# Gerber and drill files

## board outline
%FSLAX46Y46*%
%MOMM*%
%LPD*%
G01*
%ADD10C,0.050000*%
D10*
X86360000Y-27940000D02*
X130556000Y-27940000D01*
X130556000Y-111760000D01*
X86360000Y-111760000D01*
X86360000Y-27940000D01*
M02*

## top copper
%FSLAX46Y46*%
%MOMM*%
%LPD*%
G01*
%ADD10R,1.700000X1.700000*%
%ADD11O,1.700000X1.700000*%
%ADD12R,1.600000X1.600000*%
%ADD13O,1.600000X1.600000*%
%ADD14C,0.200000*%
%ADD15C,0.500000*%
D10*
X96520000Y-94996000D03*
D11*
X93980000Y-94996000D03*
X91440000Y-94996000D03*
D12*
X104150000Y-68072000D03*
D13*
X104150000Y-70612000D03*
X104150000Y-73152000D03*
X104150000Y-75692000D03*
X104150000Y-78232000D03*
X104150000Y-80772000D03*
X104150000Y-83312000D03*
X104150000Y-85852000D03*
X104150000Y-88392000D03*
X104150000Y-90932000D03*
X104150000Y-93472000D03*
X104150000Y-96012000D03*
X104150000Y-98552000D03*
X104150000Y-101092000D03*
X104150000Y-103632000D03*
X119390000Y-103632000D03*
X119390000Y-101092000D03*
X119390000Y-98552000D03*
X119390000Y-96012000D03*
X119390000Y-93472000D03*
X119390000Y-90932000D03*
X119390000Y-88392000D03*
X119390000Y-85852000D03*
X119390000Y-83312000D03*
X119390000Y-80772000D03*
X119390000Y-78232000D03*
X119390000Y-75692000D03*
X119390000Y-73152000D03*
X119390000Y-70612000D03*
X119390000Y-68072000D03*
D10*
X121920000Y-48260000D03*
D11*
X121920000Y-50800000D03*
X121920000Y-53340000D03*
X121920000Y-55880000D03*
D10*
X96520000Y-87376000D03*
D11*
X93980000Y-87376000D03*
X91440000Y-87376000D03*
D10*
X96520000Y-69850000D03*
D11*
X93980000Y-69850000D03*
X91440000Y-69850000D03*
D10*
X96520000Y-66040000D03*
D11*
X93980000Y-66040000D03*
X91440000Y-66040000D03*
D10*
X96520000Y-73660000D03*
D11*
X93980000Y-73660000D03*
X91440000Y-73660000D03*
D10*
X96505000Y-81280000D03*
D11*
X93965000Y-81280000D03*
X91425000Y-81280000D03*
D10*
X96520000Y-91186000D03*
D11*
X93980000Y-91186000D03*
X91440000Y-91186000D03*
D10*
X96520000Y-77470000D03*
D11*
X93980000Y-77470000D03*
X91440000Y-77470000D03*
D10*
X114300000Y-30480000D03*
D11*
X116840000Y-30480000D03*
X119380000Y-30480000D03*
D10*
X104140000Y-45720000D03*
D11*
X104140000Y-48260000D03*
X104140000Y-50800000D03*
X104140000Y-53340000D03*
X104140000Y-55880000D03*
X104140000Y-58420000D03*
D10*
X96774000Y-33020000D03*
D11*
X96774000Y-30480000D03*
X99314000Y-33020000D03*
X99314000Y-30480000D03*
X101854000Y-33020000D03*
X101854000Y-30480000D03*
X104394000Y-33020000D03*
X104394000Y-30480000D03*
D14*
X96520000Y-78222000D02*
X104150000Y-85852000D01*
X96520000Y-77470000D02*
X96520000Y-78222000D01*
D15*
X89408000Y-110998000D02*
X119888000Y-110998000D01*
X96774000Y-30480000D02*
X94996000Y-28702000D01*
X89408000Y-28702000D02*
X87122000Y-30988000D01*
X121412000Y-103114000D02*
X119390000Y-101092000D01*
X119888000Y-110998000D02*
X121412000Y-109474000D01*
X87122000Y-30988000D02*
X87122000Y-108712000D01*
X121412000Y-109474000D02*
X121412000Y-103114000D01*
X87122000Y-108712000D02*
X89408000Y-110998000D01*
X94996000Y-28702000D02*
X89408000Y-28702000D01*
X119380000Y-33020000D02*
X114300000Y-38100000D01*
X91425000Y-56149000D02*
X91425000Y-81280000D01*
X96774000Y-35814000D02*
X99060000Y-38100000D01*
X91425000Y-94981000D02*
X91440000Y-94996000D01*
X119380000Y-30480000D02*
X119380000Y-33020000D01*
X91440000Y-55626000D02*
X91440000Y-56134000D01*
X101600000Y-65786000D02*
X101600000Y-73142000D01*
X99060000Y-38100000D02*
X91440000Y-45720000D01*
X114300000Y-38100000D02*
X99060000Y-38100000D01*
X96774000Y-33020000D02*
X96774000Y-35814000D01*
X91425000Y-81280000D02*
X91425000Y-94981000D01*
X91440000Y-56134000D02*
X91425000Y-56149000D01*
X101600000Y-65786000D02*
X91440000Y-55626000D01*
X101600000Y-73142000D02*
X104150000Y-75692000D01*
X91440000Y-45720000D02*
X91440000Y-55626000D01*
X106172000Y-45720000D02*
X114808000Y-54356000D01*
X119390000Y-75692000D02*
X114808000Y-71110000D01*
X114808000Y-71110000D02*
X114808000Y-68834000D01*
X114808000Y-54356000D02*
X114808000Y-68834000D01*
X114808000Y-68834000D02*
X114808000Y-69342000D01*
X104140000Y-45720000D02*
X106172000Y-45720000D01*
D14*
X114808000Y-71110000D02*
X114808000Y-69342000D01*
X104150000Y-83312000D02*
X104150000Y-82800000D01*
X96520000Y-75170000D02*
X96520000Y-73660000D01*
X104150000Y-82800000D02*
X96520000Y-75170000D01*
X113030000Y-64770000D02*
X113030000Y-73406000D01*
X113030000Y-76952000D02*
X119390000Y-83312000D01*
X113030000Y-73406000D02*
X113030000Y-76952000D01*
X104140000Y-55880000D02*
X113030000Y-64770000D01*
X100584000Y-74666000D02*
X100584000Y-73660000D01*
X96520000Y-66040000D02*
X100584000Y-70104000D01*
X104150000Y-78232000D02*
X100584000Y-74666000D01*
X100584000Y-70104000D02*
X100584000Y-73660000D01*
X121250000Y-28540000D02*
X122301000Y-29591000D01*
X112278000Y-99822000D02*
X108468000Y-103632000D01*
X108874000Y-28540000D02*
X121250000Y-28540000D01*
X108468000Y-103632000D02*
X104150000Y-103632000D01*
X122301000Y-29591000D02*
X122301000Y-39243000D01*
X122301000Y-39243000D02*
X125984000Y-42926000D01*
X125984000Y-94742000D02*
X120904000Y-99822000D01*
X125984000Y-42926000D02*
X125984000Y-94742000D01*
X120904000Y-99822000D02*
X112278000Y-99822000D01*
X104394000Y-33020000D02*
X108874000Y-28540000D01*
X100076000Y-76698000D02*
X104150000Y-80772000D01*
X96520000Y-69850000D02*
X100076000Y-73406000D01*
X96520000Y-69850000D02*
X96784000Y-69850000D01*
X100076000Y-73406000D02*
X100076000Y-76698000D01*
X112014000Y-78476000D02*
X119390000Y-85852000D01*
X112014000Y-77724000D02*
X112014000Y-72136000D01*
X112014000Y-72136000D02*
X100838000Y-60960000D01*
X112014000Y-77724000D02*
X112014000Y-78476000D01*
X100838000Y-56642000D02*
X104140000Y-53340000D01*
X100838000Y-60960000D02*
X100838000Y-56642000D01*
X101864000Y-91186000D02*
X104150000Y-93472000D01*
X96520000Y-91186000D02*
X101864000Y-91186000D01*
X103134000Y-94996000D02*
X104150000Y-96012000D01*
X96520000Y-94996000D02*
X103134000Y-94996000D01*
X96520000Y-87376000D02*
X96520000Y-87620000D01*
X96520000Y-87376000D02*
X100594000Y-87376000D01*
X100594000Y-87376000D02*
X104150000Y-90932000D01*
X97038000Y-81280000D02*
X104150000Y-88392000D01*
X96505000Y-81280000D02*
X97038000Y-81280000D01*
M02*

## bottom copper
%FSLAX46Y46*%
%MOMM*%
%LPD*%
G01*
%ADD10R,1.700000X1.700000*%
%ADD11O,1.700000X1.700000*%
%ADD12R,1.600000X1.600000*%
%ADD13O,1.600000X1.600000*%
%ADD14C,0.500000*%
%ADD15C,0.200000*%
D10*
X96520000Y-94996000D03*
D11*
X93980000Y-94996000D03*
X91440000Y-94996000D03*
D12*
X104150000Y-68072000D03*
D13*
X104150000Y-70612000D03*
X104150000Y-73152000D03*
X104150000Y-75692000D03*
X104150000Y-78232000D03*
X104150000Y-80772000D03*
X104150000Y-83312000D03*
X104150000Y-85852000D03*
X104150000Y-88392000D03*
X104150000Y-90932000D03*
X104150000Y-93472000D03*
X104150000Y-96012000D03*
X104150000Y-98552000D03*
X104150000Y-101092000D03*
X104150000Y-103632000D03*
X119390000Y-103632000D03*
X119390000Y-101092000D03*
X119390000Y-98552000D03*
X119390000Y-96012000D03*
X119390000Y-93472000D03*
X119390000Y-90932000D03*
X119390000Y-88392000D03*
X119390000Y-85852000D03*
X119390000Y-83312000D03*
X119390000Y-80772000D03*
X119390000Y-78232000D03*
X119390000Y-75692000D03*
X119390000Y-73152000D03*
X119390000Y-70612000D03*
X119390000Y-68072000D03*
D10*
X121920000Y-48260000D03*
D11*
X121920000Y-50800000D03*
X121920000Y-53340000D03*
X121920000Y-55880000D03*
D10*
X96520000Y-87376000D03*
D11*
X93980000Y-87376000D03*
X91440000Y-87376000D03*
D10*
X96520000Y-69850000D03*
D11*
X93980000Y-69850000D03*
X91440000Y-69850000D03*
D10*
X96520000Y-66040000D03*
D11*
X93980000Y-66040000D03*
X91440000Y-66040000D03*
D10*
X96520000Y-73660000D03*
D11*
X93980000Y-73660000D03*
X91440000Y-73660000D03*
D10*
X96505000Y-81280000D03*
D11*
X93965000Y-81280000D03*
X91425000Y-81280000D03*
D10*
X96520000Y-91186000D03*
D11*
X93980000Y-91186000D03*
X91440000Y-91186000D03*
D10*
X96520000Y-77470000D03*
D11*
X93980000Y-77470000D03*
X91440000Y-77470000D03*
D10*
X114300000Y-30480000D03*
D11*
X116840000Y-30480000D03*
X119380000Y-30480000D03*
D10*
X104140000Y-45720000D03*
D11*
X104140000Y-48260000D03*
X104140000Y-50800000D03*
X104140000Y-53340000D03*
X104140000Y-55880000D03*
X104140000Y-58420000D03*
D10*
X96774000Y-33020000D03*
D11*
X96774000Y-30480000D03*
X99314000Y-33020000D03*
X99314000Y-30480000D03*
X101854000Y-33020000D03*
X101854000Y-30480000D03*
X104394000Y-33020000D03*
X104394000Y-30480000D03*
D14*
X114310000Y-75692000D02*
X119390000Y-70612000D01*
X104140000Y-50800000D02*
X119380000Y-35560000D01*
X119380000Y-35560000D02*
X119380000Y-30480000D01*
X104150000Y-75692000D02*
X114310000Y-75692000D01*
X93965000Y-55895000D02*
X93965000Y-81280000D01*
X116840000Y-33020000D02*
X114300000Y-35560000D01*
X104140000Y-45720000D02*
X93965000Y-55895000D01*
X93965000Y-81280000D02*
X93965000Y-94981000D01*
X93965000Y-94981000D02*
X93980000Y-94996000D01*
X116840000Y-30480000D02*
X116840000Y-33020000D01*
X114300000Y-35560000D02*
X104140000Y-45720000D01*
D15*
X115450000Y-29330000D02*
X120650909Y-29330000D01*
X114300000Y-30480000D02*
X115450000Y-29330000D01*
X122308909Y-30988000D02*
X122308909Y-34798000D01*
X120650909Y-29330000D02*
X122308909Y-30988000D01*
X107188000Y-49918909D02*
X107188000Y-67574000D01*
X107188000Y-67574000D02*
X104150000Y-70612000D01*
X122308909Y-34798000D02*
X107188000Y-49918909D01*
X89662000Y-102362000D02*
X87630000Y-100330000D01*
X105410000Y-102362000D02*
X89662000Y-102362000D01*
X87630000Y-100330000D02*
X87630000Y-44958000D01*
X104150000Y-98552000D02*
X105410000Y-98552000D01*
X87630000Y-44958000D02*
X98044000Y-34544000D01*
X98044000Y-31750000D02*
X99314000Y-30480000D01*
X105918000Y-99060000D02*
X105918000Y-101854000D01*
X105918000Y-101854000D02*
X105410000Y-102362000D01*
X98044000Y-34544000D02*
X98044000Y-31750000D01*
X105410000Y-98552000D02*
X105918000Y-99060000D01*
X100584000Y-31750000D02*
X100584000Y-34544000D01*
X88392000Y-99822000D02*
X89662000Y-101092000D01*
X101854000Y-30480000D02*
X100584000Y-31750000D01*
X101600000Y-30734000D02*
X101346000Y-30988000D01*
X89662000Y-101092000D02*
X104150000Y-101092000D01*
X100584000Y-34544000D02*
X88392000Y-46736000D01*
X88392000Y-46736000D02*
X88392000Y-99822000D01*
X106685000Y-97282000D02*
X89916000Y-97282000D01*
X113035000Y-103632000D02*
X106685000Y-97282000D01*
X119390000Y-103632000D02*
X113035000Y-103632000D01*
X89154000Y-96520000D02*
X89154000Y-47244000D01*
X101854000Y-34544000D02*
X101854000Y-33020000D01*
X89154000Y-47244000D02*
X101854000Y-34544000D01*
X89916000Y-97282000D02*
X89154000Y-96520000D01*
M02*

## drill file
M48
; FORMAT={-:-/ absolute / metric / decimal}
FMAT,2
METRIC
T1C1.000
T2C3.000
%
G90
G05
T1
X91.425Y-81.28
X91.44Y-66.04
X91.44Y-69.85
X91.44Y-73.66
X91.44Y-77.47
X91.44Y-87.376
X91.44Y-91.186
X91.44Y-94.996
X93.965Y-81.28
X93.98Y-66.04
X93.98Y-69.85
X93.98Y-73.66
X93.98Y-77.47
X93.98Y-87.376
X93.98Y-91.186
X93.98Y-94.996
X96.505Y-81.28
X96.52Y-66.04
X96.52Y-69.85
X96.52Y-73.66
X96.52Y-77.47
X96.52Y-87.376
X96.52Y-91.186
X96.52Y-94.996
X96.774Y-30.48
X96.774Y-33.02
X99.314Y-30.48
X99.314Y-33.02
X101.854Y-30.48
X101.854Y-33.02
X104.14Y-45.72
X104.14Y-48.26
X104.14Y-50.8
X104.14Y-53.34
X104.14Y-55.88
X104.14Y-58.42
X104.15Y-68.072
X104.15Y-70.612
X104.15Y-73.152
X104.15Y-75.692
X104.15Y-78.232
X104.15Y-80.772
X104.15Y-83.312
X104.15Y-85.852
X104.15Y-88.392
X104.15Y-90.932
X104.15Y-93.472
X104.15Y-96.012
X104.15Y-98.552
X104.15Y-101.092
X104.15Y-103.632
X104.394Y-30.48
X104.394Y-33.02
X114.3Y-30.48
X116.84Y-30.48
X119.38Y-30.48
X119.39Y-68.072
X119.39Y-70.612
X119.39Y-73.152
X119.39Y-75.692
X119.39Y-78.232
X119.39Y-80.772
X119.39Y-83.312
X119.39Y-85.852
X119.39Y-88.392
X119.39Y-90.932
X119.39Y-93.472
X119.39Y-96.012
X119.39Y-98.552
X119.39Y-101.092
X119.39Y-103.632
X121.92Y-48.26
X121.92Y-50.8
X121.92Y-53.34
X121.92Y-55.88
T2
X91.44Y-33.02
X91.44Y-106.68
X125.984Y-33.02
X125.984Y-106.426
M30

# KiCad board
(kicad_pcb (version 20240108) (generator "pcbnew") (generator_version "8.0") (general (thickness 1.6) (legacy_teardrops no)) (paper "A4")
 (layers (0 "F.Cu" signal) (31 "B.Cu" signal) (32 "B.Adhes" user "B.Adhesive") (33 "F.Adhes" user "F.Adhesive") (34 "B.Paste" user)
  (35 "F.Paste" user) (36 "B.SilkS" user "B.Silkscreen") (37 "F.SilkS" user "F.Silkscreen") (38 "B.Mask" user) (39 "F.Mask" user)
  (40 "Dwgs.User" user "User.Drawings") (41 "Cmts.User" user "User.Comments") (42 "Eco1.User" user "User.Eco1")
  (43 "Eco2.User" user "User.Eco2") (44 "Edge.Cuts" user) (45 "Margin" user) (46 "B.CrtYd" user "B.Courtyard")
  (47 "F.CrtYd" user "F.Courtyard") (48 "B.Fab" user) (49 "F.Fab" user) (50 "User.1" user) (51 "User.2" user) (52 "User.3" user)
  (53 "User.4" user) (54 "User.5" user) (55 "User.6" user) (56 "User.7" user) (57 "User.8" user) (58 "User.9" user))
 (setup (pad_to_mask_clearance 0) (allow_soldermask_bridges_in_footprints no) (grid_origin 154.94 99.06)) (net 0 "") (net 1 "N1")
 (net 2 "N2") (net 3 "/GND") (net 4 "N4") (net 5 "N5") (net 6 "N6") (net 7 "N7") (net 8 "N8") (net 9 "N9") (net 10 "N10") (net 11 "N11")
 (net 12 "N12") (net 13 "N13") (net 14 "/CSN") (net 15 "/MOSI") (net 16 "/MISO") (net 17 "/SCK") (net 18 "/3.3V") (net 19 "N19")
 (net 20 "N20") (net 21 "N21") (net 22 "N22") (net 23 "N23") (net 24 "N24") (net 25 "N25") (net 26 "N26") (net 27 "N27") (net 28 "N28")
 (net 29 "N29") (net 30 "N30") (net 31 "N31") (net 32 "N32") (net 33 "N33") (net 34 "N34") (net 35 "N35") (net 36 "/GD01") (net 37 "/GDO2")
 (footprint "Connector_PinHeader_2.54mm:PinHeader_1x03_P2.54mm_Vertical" (layer "F.Cu") (at 96.52 94.996 -90)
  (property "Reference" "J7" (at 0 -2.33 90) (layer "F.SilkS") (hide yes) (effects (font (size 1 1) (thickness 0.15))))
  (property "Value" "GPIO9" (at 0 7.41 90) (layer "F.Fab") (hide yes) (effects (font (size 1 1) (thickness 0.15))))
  (pad "1" thru_hole rect (at 0 0 270) (size 1.7 1.7) (drill 1) (layers "*.Cu" "*.Mask") (remove_unused_layers no) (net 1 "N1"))
  (pad "2" thru_hole oval (at 0 2.54 270) (size 1.7 1.7) (drill 1) (layers "*.Cu" "*.Mask") (remove_unused_layers no) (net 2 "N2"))
  (pad "3" thru_hole oval (at 0 5.08 270) (size 1.7 1.7) (drill 1) (layers "*.Cu" "*.Mask") (remove_unused_layers no) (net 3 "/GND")))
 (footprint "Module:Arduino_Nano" (layer "F.Cu") (at 104.15 68.072)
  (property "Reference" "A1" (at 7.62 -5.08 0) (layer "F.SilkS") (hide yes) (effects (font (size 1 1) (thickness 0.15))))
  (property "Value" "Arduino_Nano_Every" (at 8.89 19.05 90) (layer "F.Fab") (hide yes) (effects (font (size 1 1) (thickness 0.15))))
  (pad "1" thru_hole rect (at 0 0) (size 1.6 1.6) (drill 1) (layers "*.Cu" "*.Mask") (remove_unused_layers no) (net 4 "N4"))
  (pad "2" thru_hole oval (at 0 2.54) (size 1.6 1.6) (drill 1) (layers "*.Cu" "*.Mask") (remove_unused_layers no) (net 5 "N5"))
  (pad "3" thru_hole oval (at 0 5.08) (size 1.6 1.6) (drill 1) (layers "*.Cu" "*.Mask") (remove_unused_layers no) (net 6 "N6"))
  (pad "4" thru_hole oval (at 0 7.62) (size 1.6 1.6) (drill 1) (layers "*.Cu" "*.Mask") (remove_unused_layers no) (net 3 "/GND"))
  (pad "5" thru_hole oval (at 0 10.16) (size 1.6 1.6) (drill 1) (layers "*.Cu" "*.Mask") (remove_unused_layers no) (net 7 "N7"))
  (pad "6" thru_hole oval (at 0 12.7) (size 1.6 1.6) (drill 1) (layers "*.Cu" "*.Mask") (remove_unused_layers no) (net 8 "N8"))
  (pad "7" thru_hole oval (at 0 15.24) (size 1.6 1.6) (drill 1) (layers "*.Cu" "*.Mask") (remove_unused_layers no) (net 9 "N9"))
  (pad "8" thru_hole oval (at 0 17.78) (size 1.6 1.6) (drill 1) (layers "*.Cu" "*.Mask") (remove_unused_layers no) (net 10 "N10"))
  (pad "9" thru_hole oval (at 0 20.32) (size 1.6 1.6) (drill 1) (layers "*.Cu" "*.Mask") (remove_unused_layers no) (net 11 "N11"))
  (pad "10" thru_hole oval (at 0 22.86) (size 1.6 1.6) (drill 1) (layers "*.Cu" "*.Mask") (remove_unused_layers no) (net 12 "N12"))
  (pad "11" thru_hole oval (at 0 25.4) (size 1.6 1.6) (drill 1) (layers "*.Cu" "*.Mask") (remove_unused_layers no) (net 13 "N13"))
  (pad "12" thru_hole oval (at 0 27.94) (size 1.6 1.6) (drill 1) (layers "*.Cu" "*.Mask") (remove_unused_layers no) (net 1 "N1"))
  (pad "13" thru_hole oval (at 0 30.48) (size 1.6 1.6) (drill 1) (layers "*.Cu" "*.Mask") (remove_unused_layers no) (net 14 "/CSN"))
  (pad "14" thru_hole oval (at 0 33.02) (size 1.6 1.6) (drill 1) (layers "*.Cu" "*.Mask") (remove_unused_layers no) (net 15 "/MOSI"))
  (pad "15" thru_hole oval (at 0 35.56) (size 1.6 1.6) (drill 1) (layers "*.Cu" "*.Mask") (remove_unused_layers no) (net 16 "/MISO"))
  (pad "16" thru_hole oval (at 15.24 35.56) (size 1.6 1.6) (drill 1) (layers "*.Cu" "*.Mask") (remove_unused_layers no) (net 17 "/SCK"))
  (pad "17" thru_hole oval (at 15.24 33.02) (size 1.6 1.6) (drill 1) (layers "*.Cu" "*.Mask") (remove_unused_layers no) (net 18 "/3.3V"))
  (pad "18" thru_hole oval (at 15.24 30.48) (size 1.6 1.6) (drill 1) (layers "*.Cu" "*.Mask") (remove_unused_layers no) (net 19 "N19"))
  (pad "19" thru_hole oval (at 15.24 27.94) (size 1.6 1.6) (drill 1) (layers "*.Cu" "*.Mask") (remove_unused_layers no) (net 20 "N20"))
  (pad "20" thru_hole oval (at 15.24 25.4) (size 1.6 1.6) (drill 1) (layers "*.Cu" "*.Mask") (remove_unused_layers no) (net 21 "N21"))
  (pad "21" thru_hole oval (at 15.24 22.86) (size 1.6 1.6) (drill 1) (layers "*.Cu" "*.Mask") (remove_unused_layers no) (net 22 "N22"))
  (pad "22" thru_hole oval (at 15.24 20.32) (size 1.6 1.6) (drill 1) (layers "*.Cu" "*.Mask") (remove_unused_layers no) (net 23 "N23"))
  (pad "23" thru_hole oval (at 15.24 17.78) (size 1.6 1.6) (drill 1) (layers "*.Cu" "*.Mask") (remove_unused_layers no) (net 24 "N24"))
  (pad "24" thru_hole oval (at 15.24 15.24) (size 1.6 1.6) (drill 1) (layers "*.Cu" "*.Mask") (remove_unused_layers no) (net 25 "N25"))
  (pad "25" thru_hole oval (at 15.24 12.7) (size 1.6 1.6) (drill 1) (layers "*.Cu" "*.Mask") (remove_unused_layers no) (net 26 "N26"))
  (pad "26" thru_hole oval (at 15.24 10.16) (size 1.6 1.6) (drill 1) (layers "*.Cu" "*.Mask") (remove_unused_layers no) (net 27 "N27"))
  (pad "27" thru_hole oval (at 15.24 7.62) (size 1.6 1.6) (drill 1) (layers "*.Cu" "*.Mask") (remove_unused_layers no) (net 2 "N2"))
  (pad "28" thru_hole oval (at 15.24 5.08) (size 1.6 1.6) (drill 1) (layers "*.Cu" "*.Mask") (remove_unused_layers no) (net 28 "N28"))
  (pad "29" thru_hole oval (at 15.24 2.54) (size 1.6 1.6) (drill 1) (layers "*.Cu" "*.Mask") (remove_unused_layers no) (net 3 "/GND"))
  (pad "30" thru_hole oval (at 15.24 0) (size 1.6 1.6) (drill 1) (layers "*.Cu" "*.Mask") (remove_unused_layers no) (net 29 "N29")))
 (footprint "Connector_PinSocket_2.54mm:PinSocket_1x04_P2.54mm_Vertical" (layer "F.Cu") (at 121.92 48.26)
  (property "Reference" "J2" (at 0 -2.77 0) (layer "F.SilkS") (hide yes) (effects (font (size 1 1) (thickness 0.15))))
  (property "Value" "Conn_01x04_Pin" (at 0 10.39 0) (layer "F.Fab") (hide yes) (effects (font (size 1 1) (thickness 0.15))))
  (pad "1" thru_hole rect (at 0 0) (size 1.7 1.7) (drill 1) (layers "*.Cu" "*.Mask") (remove_unused_layers no) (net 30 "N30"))
  (pad "2" thru_hole oval (at 0 2.54) (size 1.7 1.7) (drill 1) (layers "*.Cu" "*.Mask") (remove_unused_layers no) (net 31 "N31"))
  (pad "3" thru_hole oval (at 0 5.08) (size 1.7 1.7) (drill 1) (layers "*.Cu" "*.Mask") (remove_unused_layers no) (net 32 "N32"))
  (pad "4" thru_hole oval (at 0 7.62) (size 1.7 1.7) (drill 1) (layers "*.Cu" "*.Mask") (remove_unused_layers no) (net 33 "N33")))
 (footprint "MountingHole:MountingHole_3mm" (layer "F.Cu") (at 91.44 33.02)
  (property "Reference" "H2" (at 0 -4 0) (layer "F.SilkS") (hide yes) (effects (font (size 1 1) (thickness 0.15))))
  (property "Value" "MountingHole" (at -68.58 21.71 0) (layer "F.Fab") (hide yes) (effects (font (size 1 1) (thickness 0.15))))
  (pad "" np_thru_hole circle (at 0 0) (size 3 3) (drill 3) (layers "*.Cu" "*.Mask")))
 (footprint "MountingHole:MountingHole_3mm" (layer "F.Cu") (at 91.44 106.68)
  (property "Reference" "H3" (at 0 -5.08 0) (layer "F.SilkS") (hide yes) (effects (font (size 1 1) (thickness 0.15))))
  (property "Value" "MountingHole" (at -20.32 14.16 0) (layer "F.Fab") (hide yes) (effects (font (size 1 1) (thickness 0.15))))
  (pad "" np_thru_hole circle (at 0 0) (size 3 3) (drill 3) (layers "*.Cu" "*.Mask")))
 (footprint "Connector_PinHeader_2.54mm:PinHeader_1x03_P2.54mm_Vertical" (layer "F.Cu") (at 96.52 87.376 -90)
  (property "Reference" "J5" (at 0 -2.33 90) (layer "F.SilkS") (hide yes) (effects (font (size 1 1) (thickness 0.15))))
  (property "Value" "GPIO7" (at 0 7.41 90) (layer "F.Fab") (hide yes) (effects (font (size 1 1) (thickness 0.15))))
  (pad "1" thru_hole rect (at 0 0 270) (size 1.7 1.7) (drill 1) (layers "*.Cu" "*.Mask") (remove_unused_layers no) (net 12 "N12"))
  (pad "2" thru_hole oval (at 0 2.54 270) (size 1.7 1.7) (drill 1) (layers "*.Cu" "*.Mask") (remove_unused_layers no) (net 2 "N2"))
  (pad "3" thru_hole oval (at 0 5.08 270) (size 1.7 1.7) (drill 1) (layers "*.Cu" "*.Mask") (remove_unused_layers no) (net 3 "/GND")))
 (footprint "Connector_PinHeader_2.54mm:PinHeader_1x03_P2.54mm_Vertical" (layer "F.Cu") (at 96.52 69.85 -90)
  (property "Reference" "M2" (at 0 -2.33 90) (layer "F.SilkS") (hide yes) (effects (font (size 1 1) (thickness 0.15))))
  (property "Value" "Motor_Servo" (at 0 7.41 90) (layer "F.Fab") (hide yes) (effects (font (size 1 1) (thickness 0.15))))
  (pad "1" thru_hole rect (at 0 0 270) (size 1.7 1.7) (drill 1) (layers "*.Cu" "*.Mask") (remove_unused_layers no) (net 8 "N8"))
  (pad "2" thru_hole oval (at 0 2.54 270) (size 1.7 1.7) (drill 1) (layers "*.Cu" "*.Mask") (remove_unused_layers no) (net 2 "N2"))
  (pad "3" thru_hole oval (at 0 5.08 270) (size 1.7 1.7) (drill 1) (layers "*.Cu" "*.Mask") (remove_unused_layers no) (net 3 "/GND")))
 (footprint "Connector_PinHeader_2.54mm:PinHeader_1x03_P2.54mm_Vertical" (layer "F.Cu") (at 96.52 66.04 -90)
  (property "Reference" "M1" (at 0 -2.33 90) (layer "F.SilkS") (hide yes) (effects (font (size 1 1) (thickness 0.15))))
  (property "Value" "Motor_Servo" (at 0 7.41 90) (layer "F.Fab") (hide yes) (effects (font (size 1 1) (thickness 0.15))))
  (pad "1" thru_hole rect (at 0 0 270) (size 1.7 1.7) (drill 1) (layers "*.Cu" "*.Mask") (remove_unused_layers no) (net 7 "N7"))
  (pad "2" thru_hole oval (at 0 2.54 270) (size 1.7 1.7) (drill 1) (layers "*.Cu" "*.Mask") (remove_unused_layers no) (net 2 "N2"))
  (pad "3" thru_hole oval (at 0 5.08 270) (size 1.7 1.7) (drill 1) (layers "*.Cu" "*.Mask") (remove_unused_layers no) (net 3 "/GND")))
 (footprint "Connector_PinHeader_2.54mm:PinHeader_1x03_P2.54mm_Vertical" (layer "F.Cu") (at 96.52 73.66 -90)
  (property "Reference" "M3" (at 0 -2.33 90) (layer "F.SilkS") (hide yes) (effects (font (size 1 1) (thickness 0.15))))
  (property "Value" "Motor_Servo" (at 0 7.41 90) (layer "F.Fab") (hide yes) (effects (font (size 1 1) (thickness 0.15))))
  (pad "1" thru_hole rect (at 0 0 270) (size 1.7 1.7) (drill 1) (layers "*.Cu" "*.Mask") (remove_unused_layers no) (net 9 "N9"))
  (pad "2" thru_hole oval (at 0 2.54 270) (size 1.7 1.7) (drill 1) (layers "*.Cu" "*.Mask") (remove_unused_layers no) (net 2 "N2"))
  (pad "3" thru_hole oval (at 0 5.08 270) (size 1.7 1.7) (drill 1) (layers "*.Cu" "*.Mask") (remove_unused_layers no) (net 3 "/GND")))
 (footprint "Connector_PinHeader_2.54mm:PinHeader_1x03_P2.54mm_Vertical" (layer "F.Cu") (at 96.505 81.28 -90)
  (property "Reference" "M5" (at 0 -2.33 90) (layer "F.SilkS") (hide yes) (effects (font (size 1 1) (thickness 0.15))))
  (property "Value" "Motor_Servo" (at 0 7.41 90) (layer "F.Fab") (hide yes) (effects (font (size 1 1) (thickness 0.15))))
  (pad "1" thru_hole rect (at 0 0 270) (size 1.7 1.7) (drill 1) (layers "*.Cu" "*.Mask") (remove_unused_layers no) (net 11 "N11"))
  (pad "2" thru_hole oval (at 0 2.54 270) (size 1.7 1.7) (drill 1) (layers "*.Cu" "*.Mask") (remove_unused_layers no) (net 2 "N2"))
  (pad "3" thru_hole oval (at 0 5.08 270) (size 1.7 1.7) (drill 1) (layers "*.Cu" "*.Mask") (remove_unused_layers no) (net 3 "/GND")))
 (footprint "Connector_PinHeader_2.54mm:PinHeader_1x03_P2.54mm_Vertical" (layer "F.Cu") (at 96.52 91.186 -90)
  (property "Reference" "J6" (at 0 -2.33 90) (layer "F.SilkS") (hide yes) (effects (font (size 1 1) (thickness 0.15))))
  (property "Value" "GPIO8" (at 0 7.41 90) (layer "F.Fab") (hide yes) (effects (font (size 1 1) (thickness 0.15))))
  (pad "1" thru_hole rect (at 0 0 270) (size 1.7 1.7) (drill 1) (layers "*.Cu" "*.Mask") (remove_unused_layers no) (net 13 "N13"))
  (pad "2" thru_hole oval (at 0 2.54 270) (size 1.7 1.7) (drill 1) (layers "*.Cu" "*.Mask") (remove_unused_layers no) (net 2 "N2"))
  (pad "3" thru_hole oval (at 0 5.08 270) (size 1.7 1.7) (drill 1) (layers "*.Cu" "*.Mask") (remove_unused_layers no) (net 3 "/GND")))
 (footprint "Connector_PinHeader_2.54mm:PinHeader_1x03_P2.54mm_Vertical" (layer "F.Cu") (at 96.52 77.47 -90)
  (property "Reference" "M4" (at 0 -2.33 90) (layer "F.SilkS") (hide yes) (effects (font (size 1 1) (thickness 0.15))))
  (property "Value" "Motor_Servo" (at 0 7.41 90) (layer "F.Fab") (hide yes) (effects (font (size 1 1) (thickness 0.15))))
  (pad "1" thru_hole rect (at 0 0 270) (size 1.7 1.7) (drill 1) (layers "*.Cu" "*.Mask") (remove_unused_layers no) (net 10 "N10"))
  (pad "2" thru_hole oval (at 0 2.54 270) (size 1.7 1.7) (drill 1) (layers "*.Cu" "*.Mask") (remove_unused_layers no) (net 2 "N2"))
  (pad "3" thru_hole oval (at 0 5.08 270) (size 1.7 1.7) (drill 1) (layers "*.Cu" "*.Mask") (remove_unused_layers no) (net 3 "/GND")))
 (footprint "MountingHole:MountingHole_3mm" (layer "F.Cu") (at 125.984 33.02)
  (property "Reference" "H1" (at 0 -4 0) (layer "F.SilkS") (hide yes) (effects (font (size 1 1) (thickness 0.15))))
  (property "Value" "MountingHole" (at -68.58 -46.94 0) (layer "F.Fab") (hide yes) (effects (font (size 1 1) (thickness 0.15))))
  (pad "" np_thru_hole circle (at 0 0) (size 3 3) (drill 3) (layers "*.Cu" "*.Mask")))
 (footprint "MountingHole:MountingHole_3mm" (layer "F.Cu") (at 125.984 106.426)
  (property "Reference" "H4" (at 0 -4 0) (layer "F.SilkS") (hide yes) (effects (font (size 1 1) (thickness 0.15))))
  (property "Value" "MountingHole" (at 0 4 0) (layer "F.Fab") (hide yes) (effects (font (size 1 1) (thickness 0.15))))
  (pad "" np_thru_hole circle (at 0 0) (size 3 3) (drill 3) (layers "*.Cu" "*.Mask")))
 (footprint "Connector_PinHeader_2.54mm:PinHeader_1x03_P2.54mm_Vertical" (layer "F.Cu") (at 114.3 30.48 90)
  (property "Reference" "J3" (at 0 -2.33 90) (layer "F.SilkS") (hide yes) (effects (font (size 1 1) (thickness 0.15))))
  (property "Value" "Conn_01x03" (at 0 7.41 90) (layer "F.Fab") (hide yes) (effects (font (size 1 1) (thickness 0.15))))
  (pad "1" thru_hole rect (at 0 0 90) (size 1.7 1.7) (drill 1) (layers "*.Cu" "*.Mask") (remove_unused_layers no) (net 5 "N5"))
  (pad "2" thru_hole oval (at 0 2.54 90) (size 1.7 1.7) (drill 1) (layers "*.Cu" "*.Mask") (remove_unused_layers no) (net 2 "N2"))
  (pad "3" thru_hole oval (at 0 5.08 90) (size 1.7 1.7) (drill 1) (layers "*.Cu" "*.Mask") (remove_unused_layers no) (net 3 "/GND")))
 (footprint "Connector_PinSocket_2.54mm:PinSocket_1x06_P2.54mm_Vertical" (layer "F.Cu") (at 104.14 45.72)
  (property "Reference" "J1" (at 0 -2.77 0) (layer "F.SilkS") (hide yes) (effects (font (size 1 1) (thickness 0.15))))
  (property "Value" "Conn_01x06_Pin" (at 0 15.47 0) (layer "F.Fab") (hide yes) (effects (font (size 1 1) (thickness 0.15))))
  (pad "1" thru_hole rect (at 0 0) (size 1.7 1.7) (drill 1) (layers "*.Cu" "*.Mask") (remove_unused_layers no) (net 2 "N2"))
  (pad "2" thru_hole oval (at 0 2.54) (size 1.7 1.7) (drill 1) (layers "*.Cu" "*.Mask") (remove_unused_layers no) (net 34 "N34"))
  (pad "3" thru_hole oval (at 0 5.08) (size 1.7 1.7) (drill 1) (layers "*.Cu" "*.Mask") (remove_unused_layers no) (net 3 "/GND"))
  (pad "4" thru_hole oval (at 0 7.62) (size 1.7 1.7) (drill 1) (layers "*.Cu" "*.Mask") (remove_unused_layers no) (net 24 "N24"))
  (pad "5" thru_hole oval (at 0 10.16) (size 1.7 1.7) (drill 1) (layers "*.Cu" "*.Mask") (remove_unused_layers no) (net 25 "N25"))
  (pad "6" thru_hole oval (at 0 12.7) (size 1.7 1.7) (drill 1) (layers "*.Cu" "*.Mask") (remove_unused_layers no) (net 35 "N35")))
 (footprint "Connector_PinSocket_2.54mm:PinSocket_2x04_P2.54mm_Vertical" (layer "B.Cu") (at 96.774 33.02 -90)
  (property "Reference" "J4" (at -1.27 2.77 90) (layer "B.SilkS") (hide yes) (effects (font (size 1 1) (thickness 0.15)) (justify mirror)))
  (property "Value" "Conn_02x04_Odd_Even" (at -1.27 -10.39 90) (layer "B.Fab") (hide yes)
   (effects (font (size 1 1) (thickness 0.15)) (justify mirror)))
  (pad "1" thru_hole rect (at 0 0 270) (size 1.7 1.7) (drill 1) (layers "*.Cu" "*.Mask") (remove_unused_layers no) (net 3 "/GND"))
  (pad "2" thru_hole oval (at -2.54 0 270) (size 1.7 1.7) (drill 1) (layers "*.Cu" "*.Mask") (remove_unused_layers no) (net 18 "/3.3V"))
  (pad "3" thru_hole oval (at 0 -2.54 270) (size 1.7 1.7) (drill 1) (layers "*.Cu" "*.Mask") (remove_unused_layers no) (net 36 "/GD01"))
  (pad "4" thru_hole oval (at -2.54 -2.54 270) (size 1.7 1.7) (drill 1) (layers "*.Cu" "*.Mask") (remove_unused_layers no) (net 14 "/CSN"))
  (pad "5" thru_hole oval (at 0 -5.08 270) (size 1.7 1.7) (drill 1) (layers "*.Cu" "*.Mask") (remove_unused_layers no) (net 17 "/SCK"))
  (pad "6" thru_hole oval (at -2.54 -5.08 270) (size 1.7 1.7) (drill 1) (layers "*.Cu" "*.Mask") (remove_unused_layers no) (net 15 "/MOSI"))
  (pad "7" thru_hole oval (at 0 -7.62 270) (size 1.7 1.7) (drill 1) (layers "*.Cu" "*.Mask") (remove_unused_layers no) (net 16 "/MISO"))
  (pad "8" thru_hole oval (at -2.54 -7.62 270) (size 1.7 1.7) (drill 1) (layers "*.Cu" "*.Mask") (remove_unused_layers no) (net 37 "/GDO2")))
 (gr_rect (start 86.36 27.94) (end 130.556 111.76) (stroke (width 0.05) (type default)) (fill none) (layer "Edge.Cuts"))
 (segment (start 96.52 78.222) (end 104.15 85.852) (width 0.2) (layer "F.Cu") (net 10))
 (segment (start 96.52 77.47) (end 96.52 78.222) (width 0.2) (layer "F.Cu") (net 10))
 (segment (start 89.408 110.998) (end 119.888 110.998) (width 0.5) (layer "F.Cu") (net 18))
 (segment (start 96.774 30.48) (end 94.996 28.702) (width 0.5) (layer "F.Cu") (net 18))
 (segment (start 89.408 28.702) (end 87.122 30.988) (width 0.5) (layer "F.Cu") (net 18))
 (segment (start 121.412 103.114) (end 119.39 101.092) (width 0.5) (layer "F.Cu") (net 18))
 (segment (start 119.888 110.998) (end 121.412 109.474) (width 0.5) (layer "F.Cu") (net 18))
 (segment (start 87.122 30.988) (end 87.122 108.712) (width 0.5) (layer "F.Cu") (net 18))
 (segment (start 121.412 109.474) (end 121.412 103.114) (width 0.5) (layer "F.Cu") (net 18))
 (segment (start 87.122 108.712) (end 89.408 110.998) (width 0.5) (layer "F.Cu") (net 18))
 (segment (start 94.996 28.702) (end 89.408 28.702) (width 0.5) (layer "F.Cu") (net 18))
 (segment (start 119.38 33.02) (end 114.3 38.1) (width 0.5) (layer "F.Cu") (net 3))
 (segment (start 91.425 56.149) (end 91.425 81.28) (width 0.5) (layer "F.Cu") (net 3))
 (segment (start 96.774 35.814) (end 99.06 38.1) (width 0.5) (layer "F.Cu") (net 3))
 (segment (start 91.425 94.981) (end 91.44 94.996) (width 0.5) (layer "F.Cu") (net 3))
 (segment (start 119.38 30.48) (end 119.38 33.02) (width 0.5) (layer "F.Cu") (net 3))
 (segment (start 91.44 55.626) (end 91.44 56.134) (width 0.5) (layer "F.Cu") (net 3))
 (segment (start 101.6 65.786) (end 101.6 73.142) (width 0.5) (layer "F.Cu") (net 3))
 (segment (start 99.06 38.1) (end 91.44 45.72) (width 0.5) (layer "F.Cu") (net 3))
 (segment (start 114.3 38.1) (end 99.06 38.1) (width 0.5) (layer "F.Cu") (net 3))
 (segment (start 96.774 33.02) (end 96.774 35.814) (width 0.5) (layer "F.Cu") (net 3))
 (segment (start 91.425 81.28) (end 91.425 94.981) (width 0.5) (layer "F.Cu") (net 3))
 (segment (start 91.44 56.134) (end 91.425 56.149) (width 0.5) (layer "F.Cu") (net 3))
 (segment (start 101.6 65.786) (end 91.44 55.626) (width 0.5) (layer "F.Cu") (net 3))
 (segment (start 101.6 73.142) (end 104.15 75.692) (width 0.5) (layer "F.Cu") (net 3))
 (segment (start 91.44 45.72) (end 91.44 55.626) (width 0.5) (layer "F.Cu") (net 3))
 (segment (start 114.31 75.692) (end 119.39 70.612) (width 0.5) (layer "B.Cu") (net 3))
 (segment (start 104.14 50.8) (end 119.38 35.56) (width 0.5) (layer "B.Cu") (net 3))
 (segment (start 119.38 35.56) (end 119.38 30.48) (width 0.5) (layer "B.Cu") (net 3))
 (segment (start 104.15 75.692) (end 114.31 75.692) (width 0.5) (layer "B.Cu") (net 3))
 (segment (start 106.172 45.72) (end 114.808 54.356) (width 0.5) (layer "F.Cu") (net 2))
 (segment (start 119.39 75.692) (end 114.808 71.11) (width 0.5) (layer "F.Cu") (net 2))
 (segment (start 114.808 71.11) (end 114.808 68.834) (width 0.5) (layer "F.Cu") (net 2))
 (segment (start 114.808 54.356) (end 114.808 68.834) (width 0.5) (layer "F.Cu") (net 2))
 (segment (start 114.808 68.834) (end 114.808 69.342) (width 0.5) (layer "F.Cu") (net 2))
 (segment (start 104.14 45.72) (end 106.172 45.72) (width 0.5) (layer "F.Cu") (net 2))
 (segment (start 114.808 71.11) (end 114.808 69.342) (width 0.2) (layer "F.Cu") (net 2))
 (segment (start 93.965 55.895) (end 93.965 81.28) (width 0.5) (layer "B.Cu") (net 2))
 (segment (start 116.84 33.02) (end 114.3 35.56) (width 0.5) (layer "B.Cu") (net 2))
 (segment (start 104.14 45.72) (end 93.965 55.895) (width 0.5) (layer "B.Cu") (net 2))
 (segment (start 93.965 81.28) (end 93.965 94.981) (width 0.5) (layer "B.Cu") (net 2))
 (segment (start 93.965 94.981) (end 93.98 94.996) (width 0.5) (layer "B.Cu") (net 2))
 (segment (start 116.84 30.48) (end 116.84 33.02) (width 0.5) (layer "B.Cu") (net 2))
 (segment (start 114.3 35.56) (end 104.14 45.72) (width 0.5) (layer "B.Cu") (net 2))
 (segment (start 104.15 83.312) (end 104.15 82.8) (width 0.2) (layer "F.Cu") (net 9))
 (segment (start 96.52 75.17) (end 96.52 73.66) (width 0.2) (layer "F.Cu") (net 9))
 (segment (start 104.15 82.8) (end 96.52 75.17) (width 0.2) (layer "F.Cu") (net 9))
 (segment (start 113.03 64.77) (end 113.03 73.406) (width 0.2) (layer "F.Cu") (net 25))
 (segment (start 113.03 76.952) (end 119.39 83.312) (width 0.2) (layer "F.Cu") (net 25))
 (segment (start 113.03 73.406) (end 113.03 76.952) (width 0.2) (layer "F.Cu") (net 25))
 (segment (start 104.14 55.88) (end 113.03 64.77) (width 0.2) (layer "F.Cu") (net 25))
 (segment (start 100.584 74.666) (end 100.584 73.66) (width 0.2) (layer "F.Cu") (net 7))
 (segment (start 96.52 66.04) (end 100.584 70.104) (width 0.2) (layer "F.Cu") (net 7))
 (segment (start 104.15 78.232) (end 100.584 74.666) (width 0.2) (layer "F.Cu") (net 7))
 (segment (start 100.584 70.104) (end 100.584 73.66) (width 0.2) (layer "F.Cu") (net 7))
 (segment (start 115.45 29.33) (end 120.650909 29.33) (width 0.2) (layer "B.Cu") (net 5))
 (segment (start 114.3 30.48) (end 115.45 29.33) (width 0.2) (layer "B.Cu") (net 5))
 (segment (start 122.308909 30.988) (end 122.308909 34.798) (width 0.2) (layer "B.Cu") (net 5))
 (segment (start 120.650909 29.33) (end 122.308909 30.988) (width 0.2) (layer "B.Cu") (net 5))
 (segment (start 107.188 49.918909) (end 107.188 67.574) (width 0.2) (layer "B.Cu") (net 5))
 (segment (start 107.188 67.574) (end 104.15 70.612) (width 0.2) (layer "B.Cu") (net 5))
 (segment (start 122.308909 34.798) (end 107.188 49.918909) (width 0.2) (layer "B.Cu") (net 5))
 (segment (start 121.25 28.54) (end 122.301 29.591) (width 0.2) (layer "F.Cu") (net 16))
 (segment (start 112.278 99.822) (end 108.468 103.632) (width 0.2) (layer "F.Cu") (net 16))
 (segment (start 108.874 28.54) (end 121.25 28.54) (width 0.2) (layer "F.Cu") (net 16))
 (segment (start 108.468 103.632) (end 104.15 103.632) (width 0.2) (layer "F.Cu") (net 16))
 (segment (start 122.301 29.591) (end 122.301 39.243) (width 0.2) (layer "F.Cu") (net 16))
 (segment (start 122.301 39.243) (end 125.984 42.926) (width 0.2) (layer "F.Cu") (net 16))
 (segment (start 125.984 94.742) (end 120.904 99.822) (width 0.2) (layer "F.Cu") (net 16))
 (segment (start 125.984 42.926) (end 125.984 94.742) (width 0.2) (layer "F.Cu") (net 16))
 (segment (start 120.904 99.822) (end 112.278 99.822) (width 0.2) (layer "F.Cu") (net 16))
 (segment (start 104.394 33.02) (end 108.874 28.54) (width 0.2) (layer "F.Cu") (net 16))
 (segment (start 89.662 102.362) (end 87.63 100.33) (width 0.2) (layer "B.Cu") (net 14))
 (segment (start 105.41 102.362) (end 89.662 102.362) (width 0.2) (layer "B.Cu") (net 14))
 (segment (start 87.63 100.33) (end 87.63 44.958) (width 0.2) (layer "B.Cu") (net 14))
 (segment (start 104.15 98.552) (end 105.41 98.552) (width 0.2) (layer "B.Cu") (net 14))
 (segment (start 87.63 44.958) (end 98.044 34.544) (width 0.2) (layer "B.Cu") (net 14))
 (segment (start 98.044 31.75) (end 99.314 30.48) (width 0.2) (layer "B.Cu") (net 14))
 (segment (start 105.918 99.06) (end 105.918 101.854) (width 0.2) (layer "B.Cu") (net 14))
 (segment (start 105.918 101.854) (end 105.41 102.362) (width 0.2) (layer "B.Cu") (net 14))
 (segment (start 98.044 34.544) (end 98.044 31.75) (width 0.2) (layer "B.Cu") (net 14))
 (segment (start 105.41 98.552) (end 105.918 99.06) (width 0.2) (layer "B.Cu") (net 14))
 (segment (start 100.076 76.698) (end 104.15 80.772) (width 0.2) (layer "F.Cu") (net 8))
 (segment (start 96.52 69.85) (end 100.076 73.406) (width 0.2) (layer "F.Cu") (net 8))
 (segment (start 96.52 69.85) (end 96.784 69.85) (width 0.2) (layer "F.Cu") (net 8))
 (segment (start 100.076 73.406) (end 100.076 76.698) (width 0.2) (layer "F.Cu") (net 8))
 (segment (start 112.014 78.476) (end 119.39 85.852) (width 0.2) (layer "F.Cu") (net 24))
 (segment (start 112.014 77.724) (end 112.014 72.136) (width 0.2) (layer "F.Cu") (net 24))
 (segment (start 112.014 72.136) (end 100.838 60.96) (width 0.2) (layer "F.Cu") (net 24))
 (segment (start 112.014 77.724) (end 112.014 78.476) (width 0.2) (layer "F.Cu") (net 24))
 (segment (start 100.838 56.642) (end 104.14 53.34) (width 0.2) (layer "F.Cu") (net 24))
 (segment (start 100.838 60.96) (end 100.838 56.642) (width 0.2) (layer "F.Cu") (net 24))
 (segment (start 100.584 31.75) (end 100.584 34.544) (width 0.2) (layer "B.Cu") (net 15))
 (segment (start 88.392 99.822) (end 89.662 101.092) (width 0.2) (layer "B.Cu") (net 15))
 (segment (start 101.854 30.48) (end 100.584 31.75) (width 0.2) (layer "B.Cu") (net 15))
 (segment (start 101.6 30.734) (end 101.346 30.988) (width 0.2) (layer "B.Cu") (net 15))
 (segment (start 89.662 101.092) (end 104.15 101.092) (width 0.2) (layer "B.Cu") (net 15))
 (segment (start 100.584 34.544) (end 88.392 46.736) (width 0.2) (layer "B.Cu") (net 15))
 (segment (start 88.392 46.736) (end 88.392 99.822) (width 0.2) (layer "B.Cu") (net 15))
 (segment (start 101.864 91.186) (end 104.15 93.472) (width 0.2) (layer "F.Cu") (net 13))
 (segment (start 96.52 91.186) (end 101.864 91.186) (width 0.2) (layer "F.Cu") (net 13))
 (segment (start 103.134 94.996) (end 104.15 96.012) (width 0.2) (layer "F.Cu") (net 1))
 (segment (start 96.52 94.996) (end 103.134 94.996) (width 0.2) (layer "F.Cu") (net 1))
 (segment (start 96.52 87.376) (end 96.52 87.62) (width 0.2) (layer "F.Cu") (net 12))
 (segment (start 96.52 87.376) (end 100.594 87.376) (width 0.2) (layer "F.Cu") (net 12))
 (segment (start 100.594 87.376) (end 104.15 90.932) (width 0.2) (layer "F.Cu") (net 12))
 (segment (start 106.685 97.282) (end 89.916 97.282) (width 0.2) (layer "B.Cu") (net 17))
 (segment (start 113.035 103.632) (end 106.685 97.282) (width 0.2) (layer "B.Cu") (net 17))
 (segment (start 119.39 103.632) (end 113.035 103.632) (width 0.2) (layer "B.Cu") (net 17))
 (segment (start 89.154 96.52) (end 89.154 47.244) (width 0.2) (layer "B.Cu") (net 17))
 (segment (start 101.854 34.544) (end 101.854 33.02) (width 0.2) (layer "B.Cu") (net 17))
 (segment (start 89.154 47.244) (end 101.854 34.544) (width 0.2) (layer "B.Cu") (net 17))
 (segment (start 89.916 97.282) (end 89.154 96.52) (width 0.2) (layer "B.Cu") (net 17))
 (segment (start 97.038 81.28) (end 104.15 88.392) (width 0.2) (layer "F.Cu") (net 11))
 (segment (start 96.505 81.28) (end 97.038 81.28) (width 0.2) (layer "F.Cu") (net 11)))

